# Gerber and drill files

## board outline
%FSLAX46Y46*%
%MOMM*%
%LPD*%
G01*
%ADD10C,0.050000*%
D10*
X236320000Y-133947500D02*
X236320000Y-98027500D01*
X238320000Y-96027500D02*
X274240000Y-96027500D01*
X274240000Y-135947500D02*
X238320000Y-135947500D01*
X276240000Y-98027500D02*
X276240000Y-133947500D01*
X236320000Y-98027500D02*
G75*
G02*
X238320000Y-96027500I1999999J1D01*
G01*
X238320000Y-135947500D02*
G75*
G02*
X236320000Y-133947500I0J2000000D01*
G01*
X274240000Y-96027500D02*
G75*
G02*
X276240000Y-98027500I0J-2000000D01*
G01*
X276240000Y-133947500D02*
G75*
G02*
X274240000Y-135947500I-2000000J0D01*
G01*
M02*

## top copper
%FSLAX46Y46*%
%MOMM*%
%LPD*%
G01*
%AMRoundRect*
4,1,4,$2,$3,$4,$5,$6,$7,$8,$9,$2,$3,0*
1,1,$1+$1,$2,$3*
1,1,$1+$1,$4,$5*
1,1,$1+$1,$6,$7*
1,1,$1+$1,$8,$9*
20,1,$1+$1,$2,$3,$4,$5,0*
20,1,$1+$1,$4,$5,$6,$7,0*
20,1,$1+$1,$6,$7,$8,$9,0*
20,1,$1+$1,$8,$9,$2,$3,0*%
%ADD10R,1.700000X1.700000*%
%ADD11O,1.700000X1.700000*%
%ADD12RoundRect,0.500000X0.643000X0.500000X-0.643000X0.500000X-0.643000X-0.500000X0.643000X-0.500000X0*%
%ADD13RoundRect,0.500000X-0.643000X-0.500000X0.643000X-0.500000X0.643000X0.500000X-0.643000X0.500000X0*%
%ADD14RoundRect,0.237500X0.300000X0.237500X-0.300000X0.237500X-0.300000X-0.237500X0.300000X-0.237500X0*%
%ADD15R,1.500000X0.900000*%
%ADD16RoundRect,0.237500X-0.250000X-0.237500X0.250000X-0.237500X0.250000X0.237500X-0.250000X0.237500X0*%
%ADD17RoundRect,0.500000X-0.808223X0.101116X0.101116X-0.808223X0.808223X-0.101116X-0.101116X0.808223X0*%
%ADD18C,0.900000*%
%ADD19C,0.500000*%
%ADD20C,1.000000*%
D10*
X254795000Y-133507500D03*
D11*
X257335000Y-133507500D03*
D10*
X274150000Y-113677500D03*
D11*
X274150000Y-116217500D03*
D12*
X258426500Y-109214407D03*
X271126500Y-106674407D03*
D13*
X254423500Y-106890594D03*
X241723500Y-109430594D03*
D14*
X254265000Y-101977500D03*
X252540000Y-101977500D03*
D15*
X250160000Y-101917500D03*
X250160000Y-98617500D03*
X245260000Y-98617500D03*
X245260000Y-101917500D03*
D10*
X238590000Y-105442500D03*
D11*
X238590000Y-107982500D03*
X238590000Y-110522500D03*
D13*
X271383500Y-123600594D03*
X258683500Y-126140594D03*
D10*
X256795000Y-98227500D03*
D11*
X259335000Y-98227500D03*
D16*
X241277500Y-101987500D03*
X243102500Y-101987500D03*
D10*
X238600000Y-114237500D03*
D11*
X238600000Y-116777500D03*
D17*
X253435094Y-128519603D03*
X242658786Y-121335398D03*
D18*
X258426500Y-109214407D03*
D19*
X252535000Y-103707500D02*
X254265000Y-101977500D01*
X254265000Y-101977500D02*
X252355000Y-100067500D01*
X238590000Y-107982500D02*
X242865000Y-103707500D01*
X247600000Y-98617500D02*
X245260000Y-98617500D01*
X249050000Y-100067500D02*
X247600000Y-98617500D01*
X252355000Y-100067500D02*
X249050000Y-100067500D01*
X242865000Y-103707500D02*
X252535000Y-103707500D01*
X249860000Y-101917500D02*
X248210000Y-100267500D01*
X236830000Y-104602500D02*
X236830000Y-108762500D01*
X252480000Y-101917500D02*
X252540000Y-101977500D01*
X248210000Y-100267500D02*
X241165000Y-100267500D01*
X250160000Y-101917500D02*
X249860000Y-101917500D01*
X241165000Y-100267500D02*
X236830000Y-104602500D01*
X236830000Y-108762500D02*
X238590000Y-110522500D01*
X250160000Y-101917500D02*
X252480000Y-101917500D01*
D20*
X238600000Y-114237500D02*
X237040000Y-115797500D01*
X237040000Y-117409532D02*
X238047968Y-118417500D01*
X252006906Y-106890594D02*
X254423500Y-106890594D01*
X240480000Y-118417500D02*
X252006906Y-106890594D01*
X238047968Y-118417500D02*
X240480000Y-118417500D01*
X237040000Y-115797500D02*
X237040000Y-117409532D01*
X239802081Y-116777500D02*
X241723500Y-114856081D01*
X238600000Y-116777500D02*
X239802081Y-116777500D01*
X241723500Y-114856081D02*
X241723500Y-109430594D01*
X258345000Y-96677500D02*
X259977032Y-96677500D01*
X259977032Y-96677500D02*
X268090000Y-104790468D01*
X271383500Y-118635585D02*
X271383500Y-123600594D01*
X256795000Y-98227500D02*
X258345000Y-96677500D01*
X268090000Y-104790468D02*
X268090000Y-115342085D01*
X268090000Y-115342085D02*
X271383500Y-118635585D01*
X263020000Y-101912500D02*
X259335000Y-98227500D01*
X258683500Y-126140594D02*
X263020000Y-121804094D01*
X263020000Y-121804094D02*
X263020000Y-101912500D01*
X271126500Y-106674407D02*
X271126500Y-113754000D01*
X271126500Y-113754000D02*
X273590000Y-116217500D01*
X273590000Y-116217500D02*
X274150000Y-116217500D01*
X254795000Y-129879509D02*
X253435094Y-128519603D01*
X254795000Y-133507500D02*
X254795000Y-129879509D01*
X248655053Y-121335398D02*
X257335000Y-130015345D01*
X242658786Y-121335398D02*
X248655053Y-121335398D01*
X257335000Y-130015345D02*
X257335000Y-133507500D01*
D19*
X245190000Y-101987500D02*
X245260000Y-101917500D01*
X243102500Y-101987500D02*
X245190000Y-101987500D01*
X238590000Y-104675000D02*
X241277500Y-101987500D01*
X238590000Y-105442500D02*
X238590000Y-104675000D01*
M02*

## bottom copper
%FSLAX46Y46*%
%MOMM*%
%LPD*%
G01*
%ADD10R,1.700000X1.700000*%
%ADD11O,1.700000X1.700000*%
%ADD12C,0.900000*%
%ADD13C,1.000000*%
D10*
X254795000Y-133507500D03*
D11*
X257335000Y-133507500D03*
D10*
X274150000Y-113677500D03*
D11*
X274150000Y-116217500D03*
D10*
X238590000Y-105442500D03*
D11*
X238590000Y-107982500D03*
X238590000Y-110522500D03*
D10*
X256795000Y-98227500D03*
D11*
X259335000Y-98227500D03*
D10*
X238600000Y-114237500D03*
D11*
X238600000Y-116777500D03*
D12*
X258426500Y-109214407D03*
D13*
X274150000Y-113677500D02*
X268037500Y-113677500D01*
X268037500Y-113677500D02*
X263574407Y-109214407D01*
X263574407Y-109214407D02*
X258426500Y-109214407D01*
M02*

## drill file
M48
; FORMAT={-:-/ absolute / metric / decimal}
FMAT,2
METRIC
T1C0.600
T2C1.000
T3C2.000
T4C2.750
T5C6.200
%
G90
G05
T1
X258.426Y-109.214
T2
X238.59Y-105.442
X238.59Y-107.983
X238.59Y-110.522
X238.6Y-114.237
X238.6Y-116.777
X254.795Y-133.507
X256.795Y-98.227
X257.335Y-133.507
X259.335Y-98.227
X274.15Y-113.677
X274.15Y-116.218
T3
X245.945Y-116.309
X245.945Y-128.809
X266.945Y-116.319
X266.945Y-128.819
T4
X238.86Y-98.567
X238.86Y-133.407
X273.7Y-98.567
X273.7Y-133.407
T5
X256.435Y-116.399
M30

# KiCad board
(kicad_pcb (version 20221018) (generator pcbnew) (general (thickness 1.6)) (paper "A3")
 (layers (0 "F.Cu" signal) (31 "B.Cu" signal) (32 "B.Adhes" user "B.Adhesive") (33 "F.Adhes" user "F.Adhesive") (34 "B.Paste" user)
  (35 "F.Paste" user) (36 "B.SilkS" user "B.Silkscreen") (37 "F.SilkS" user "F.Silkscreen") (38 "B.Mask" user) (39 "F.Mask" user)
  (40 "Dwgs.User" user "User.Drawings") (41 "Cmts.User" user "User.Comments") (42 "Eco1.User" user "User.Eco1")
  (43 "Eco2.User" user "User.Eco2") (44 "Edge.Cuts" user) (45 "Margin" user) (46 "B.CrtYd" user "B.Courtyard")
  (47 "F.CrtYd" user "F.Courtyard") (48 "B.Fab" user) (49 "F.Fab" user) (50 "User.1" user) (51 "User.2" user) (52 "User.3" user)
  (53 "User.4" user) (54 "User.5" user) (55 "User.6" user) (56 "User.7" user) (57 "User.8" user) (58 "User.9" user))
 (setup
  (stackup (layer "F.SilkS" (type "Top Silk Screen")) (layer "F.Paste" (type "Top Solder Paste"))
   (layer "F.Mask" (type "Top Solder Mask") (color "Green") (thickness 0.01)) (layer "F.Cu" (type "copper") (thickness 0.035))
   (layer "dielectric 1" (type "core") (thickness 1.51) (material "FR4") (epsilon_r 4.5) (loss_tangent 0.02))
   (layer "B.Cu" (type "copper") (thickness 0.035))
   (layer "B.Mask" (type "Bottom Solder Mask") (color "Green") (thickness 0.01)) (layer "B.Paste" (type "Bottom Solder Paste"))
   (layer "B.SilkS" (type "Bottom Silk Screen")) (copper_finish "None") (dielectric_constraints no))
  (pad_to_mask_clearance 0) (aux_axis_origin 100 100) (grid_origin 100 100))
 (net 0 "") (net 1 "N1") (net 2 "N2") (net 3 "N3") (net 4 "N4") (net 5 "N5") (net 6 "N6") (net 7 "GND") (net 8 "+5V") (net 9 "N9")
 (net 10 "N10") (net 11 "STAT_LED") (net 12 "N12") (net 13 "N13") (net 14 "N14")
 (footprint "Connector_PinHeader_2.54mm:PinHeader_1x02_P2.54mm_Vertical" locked (layer "F.Cu") (at 254.795 133.5075 90)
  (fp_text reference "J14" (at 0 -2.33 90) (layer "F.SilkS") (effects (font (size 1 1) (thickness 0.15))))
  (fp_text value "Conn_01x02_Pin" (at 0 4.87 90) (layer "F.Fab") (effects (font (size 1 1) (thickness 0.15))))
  (pad "1" thru_hole rect locked (at 0 0 90) (size 1.7 1.7) (drill 1) (layers "*.Cu" "*.Mask") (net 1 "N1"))
  (pad "2" thru_hole oval locked (at 0 2.54 90) (size 1.7 1.7) (drill 1) (layers "*.Cu" "*.Mask") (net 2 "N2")))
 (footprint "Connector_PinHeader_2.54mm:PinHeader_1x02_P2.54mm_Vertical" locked (layer "F.Cu") (at 274.15 113.6775)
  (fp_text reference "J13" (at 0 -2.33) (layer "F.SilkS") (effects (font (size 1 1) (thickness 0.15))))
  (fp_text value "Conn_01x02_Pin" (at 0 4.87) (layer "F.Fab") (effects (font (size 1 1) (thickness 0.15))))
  (pad "1" thru_hole rect locked (at 0 0) (size 1.7 1.7) (drill 1) (layers "*.Cu" "*.Mask") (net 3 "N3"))
  (pad "2" thru_hole oval locked (at 0 2.54) (size 1.7 1.7) (drill 1) (layers "*.Cu" "*.Mask") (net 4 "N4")))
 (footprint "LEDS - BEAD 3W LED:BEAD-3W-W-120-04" (layer "F.Cu") (at 273.6665 104.134407 180)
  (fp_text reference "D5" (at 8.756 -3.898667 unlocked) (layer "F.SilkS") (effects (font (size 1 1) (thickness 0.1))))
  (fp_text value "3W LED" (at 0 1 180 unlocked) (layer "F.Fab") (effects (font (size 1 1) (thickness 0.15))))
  (pad "1" smd roundrect (at 15.24 -5.08 180) (size 2.286 2) (layers "F.Cu" "F.Paste" "F.Mask") (roundrect_rratio 0.25) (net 3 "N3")
   (thermal_bridge_angle 45))
  (pad "2" smd roundrect (at 2.54 -2.54 180) (size 2.286 2) (layers "F.Cu" "F.Paste" "F.Mask") (roundrect_rratio 0.25) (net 4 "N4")
   (thermal_bridge_angle 45)))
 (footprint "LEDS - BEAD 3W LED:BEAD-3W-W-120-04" (layer "F.Cu") (at 239.1835 111.970594)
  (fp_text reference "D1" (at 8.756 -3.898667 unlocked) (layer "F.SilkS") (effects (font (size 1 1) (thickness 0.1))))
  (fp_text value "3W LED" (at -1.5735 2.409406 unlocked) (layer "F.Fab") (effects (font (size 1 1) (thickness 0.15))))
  (pad "1" smd roundrect (at 15.24 -5.08) (size 2.286 2) (layers "F.Cu" "F.Paste" "F.Mask") (roundrect_rratio 0.25) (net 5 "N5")
   (thermal_bridge_angle 45))
  (pad "2" smd roundrect (at 2.54 -2.54) (size 2.286 2) (layers "F.Cu" "F.Paste" "F.Mask") (roundrect_rratio 0.25) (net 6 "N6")
   (thermal_bridge_angle 45)))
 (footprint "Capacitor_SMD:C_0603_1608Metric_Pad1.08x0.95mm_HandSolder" (layer "F.Cu") (at 253.4025 101.9775 180)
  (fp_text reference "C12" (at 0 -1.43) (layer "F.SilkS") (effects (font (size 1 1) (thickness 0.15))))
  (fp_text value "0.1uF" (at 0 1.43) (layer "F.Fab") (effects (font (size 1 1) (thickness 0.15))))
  (pad "1" smd roundrect (at -0.8625 0 180) (size 1.075 0.95) (layers "F.Cu" "F.Paste" "F.Mask") (roundrect_rratio 0.25) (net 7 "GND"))
  (pad "2" smd roundrect (at 0.8625 0 180) (size 1.075 0.95) (layers "F.Cu" "F.Paste" "F.Mask") (roundrect_rratio 0.25) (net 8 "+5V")))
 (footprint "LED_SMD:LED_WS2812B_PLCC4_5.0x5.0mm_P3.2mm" (layer "F.Cu") (at 247.71 100.2675 180)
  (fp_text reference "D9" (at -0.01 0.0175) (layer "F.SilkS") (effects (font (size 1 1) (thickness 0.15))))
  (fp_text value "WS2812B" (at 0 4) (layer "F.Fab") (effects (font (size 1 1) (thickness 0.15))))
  (pad "1" smd rect (at -2.45 -1.65 180) (size 1.5 0.9) (layers "F.Cu" "F.Paste" "F.Mask") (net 8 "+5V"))
  (pad "2" smd rect (at -2.45 1.65 180) (size 1.5 0.9) (layers "F.Cu" "F.Paste" "F.Mask") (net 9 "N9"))
  (pad "3" smd rect (at 2.45 1.65 180) (size 1.5 0.9) (layers "F.Cu" "F.Paste" "F.Mask") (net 7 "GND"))
  (pad "4" smd rect (at 2.45 -1.65 180) (size 1.5 0.9) (layers "F.Cu" "F.Paste" "F.Mask") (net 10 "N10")))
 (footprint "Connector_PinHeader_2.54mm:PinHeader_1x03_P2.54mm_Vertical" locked (layer "F.Cu") (at 238.59 105.4425)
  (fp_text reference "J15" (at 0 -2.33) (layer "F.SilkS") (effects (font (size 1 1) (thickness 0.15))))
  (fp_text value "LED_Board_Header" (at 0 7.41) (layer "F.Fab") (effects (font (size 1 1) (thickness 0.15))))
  (pad "1" thru_hole rect locked (at 0 0) (size 1.7 1.7) (drill 1) (layers "*.Cu" "*.Mask") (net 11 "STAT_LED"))
  (pad "2" thru_hole oval locked (at 0 2.54) (size 1.7 1.7) (drill 1) (layers "*.Cu" "*.Mask") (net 7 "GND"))
  (pad "3" thru_hole oval locked (at 0 5.08) (size 1.7 1.7) (drill 1) (layers "*.Cu" "*.Mask") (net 8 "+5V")))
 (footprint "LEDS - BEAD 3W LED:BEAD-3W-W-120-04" (layer "F.Cu") (at 256.1435 128.680594)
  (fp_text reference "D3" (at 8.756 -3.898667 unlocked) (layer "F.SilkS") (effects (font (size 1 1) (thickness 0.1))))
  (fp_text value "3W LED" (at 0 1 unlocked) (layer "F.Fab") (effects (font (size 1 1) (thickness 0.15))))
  (pad "1" smd roundrect (at 15.24 -5.08) (size 2.286 2) (layers "F.Cu" "F.Paste" "F.Mask") (roundrect_rratio 0.25) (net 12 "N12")
   (thermal_bridge_angle 45))
  (pad "2" smd roundrect (at 2.54 -2.54) (size 2.286 2) (layers "F.Cu" "F.Paste" "F.Mask") (roundrect_rratio 0.25) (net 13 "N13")
   (thermal_bridge_angle 45)))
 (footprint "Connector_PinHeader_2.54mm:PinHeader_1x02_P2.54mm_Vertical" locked (layer "F.Cu") (at 256.795 98.2275 90)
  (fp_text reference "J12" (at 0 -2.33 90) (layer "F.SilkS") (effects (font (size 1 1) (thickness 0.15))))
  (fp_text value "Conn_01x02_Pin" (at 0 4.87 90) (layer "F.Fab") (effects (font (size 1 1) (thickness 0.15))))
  (pad "1" thru_hole rect locked (at 0 0 90) (size 1.7 1.7) (drill 1) (layers "*.Cu" "*.Mask") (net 12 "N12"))
  (pad "2" thru_hole oval locked (at 0 2.54 90) (size 1.7 1.7) (drill 1) (layers "*.Cu" "*.Mask") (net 13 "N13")))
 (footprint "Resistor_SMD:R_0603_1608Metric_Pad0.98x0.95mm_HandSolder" (layer "F.Cu") (at 242.19 101.9875)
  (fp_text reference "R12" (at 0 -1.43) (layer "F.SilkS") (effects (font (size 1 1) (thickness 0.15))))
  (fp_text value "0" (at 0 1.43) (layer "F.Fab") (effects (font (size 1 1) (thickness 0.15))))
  (pad "1" smd roundrect (at -0.9125 0) (size 0.975 0.95) (layers "F.Cu" "F.Paste" "F.Mask") (roundrect_rratio 0.25) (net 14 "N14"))
  (pad "2" smd roundrect (at 0.9125 0) (size 0.975 0.95) (layers "F.Cu" "F.Paste" "F.Mask") (roundrect_rratio 0.25) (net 10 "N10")))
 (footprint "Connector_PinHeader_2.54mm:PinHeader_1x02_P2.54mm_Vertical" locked (layer "F.Cu") (at 238.6 114.2375)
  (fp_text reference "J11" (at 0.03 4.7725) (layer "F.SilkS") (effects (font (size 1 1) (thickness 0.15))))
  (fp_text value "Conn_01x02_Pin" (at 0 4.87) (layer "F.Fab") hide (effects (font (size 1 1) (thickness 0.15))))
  (pad "1" thru_hole rect locked (at 0 0) (size 1.7 1.7) (drill 1) (layers "*.Cu" "*.Mask") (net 5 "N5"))
  (pad "2" thru_hole oval locked (at 0 2.54) (size 1.7 1.7) (drill 1) (layers "*.Cu" "*.Mask") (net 6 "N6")))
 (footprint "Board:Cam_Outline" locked (layer "F.Cu") (at 236.32 96.0275)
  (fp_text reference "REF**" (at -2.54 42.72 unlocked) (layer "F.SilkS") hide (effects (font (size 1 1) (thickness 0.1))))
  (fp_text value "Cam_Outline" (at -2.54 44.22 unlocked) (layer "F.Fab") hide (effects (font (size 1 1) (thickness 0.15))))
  (fp_line (start 0 37.92) (end 0 2) (stroke (width 0.05) (type default)) (layer "Edge.Cuts"))
  (fp_line (start 2 0) (end 37.92 0) (stroke (width 0.05) (type default)) (layer "Edge.Cuts"))
  (fp_line (start 37.92 39.92) (end 2 39.92) (stroke (width 0.05) (type default)) (layer "Edge.Cuts"))
  (fp_line (start 39.92 2) (end 39.92 37.92) (stroke (width 0.05) (type default)) (layer "Edge.Cuts"))
  (fp_arc (start 0 2) (mid 0.585786 0.585786) (end 2 0) (stroke (width 0.05) (type default)) (layer "Edge.Cuts"))
  (fp_arc (start 2 39.92) (mid 0.585786 39.334214) (end 0 37.92) (stroke (width 0.05) (type default)) (layer "Edge.Cuts"))
  (fp_arc (start 37.92 0) (mid 39.334214 0.585786) (end 39.92 2) (stroke (width 0.05) (type default)) (layer "Edge.Cuts"))
  (fp_arc (start 39.92 37.92) (mid 39.334214 39.334214) (end 37.92 39.92) (stroke (width 0.05) (type default)) (layer "Edge.Cuts"))
  (pad "" np_thru_hole circle locked (at 2.54 2.54) (size 2.75 2.75) (drill 2.75) (layers "F&B.Cu" "*.Mask"))
  (pad "" np_thru_hole circle locked (at 2.54 37.38) (size 2.75 2.75) (drill 2.75) (layers "F&B.Cu" "*.Mask"))
  (pad "" np_thru_hole circle locked (at 9.625174 20.281079) (size 2 2) (drill 2) (layers "F&B.Cu" "*.Mask"))
  (pad "" np_thru_hole circle locked (at 9.625174 32.781079) (size 2 2) (drill 2) (layers "F&B.Cu" "*.Mask"))
  (pad "" np_thru_hole circle locked (at 20.115174 20.371079) (size 6.2 6.2) (drill 6.2) (layers "F&B.Cu" "*.Mask"))
  (pad "" np_thru_hole circle locked (at 30.625174 20.291079) (size 2 2) (drill 2) (layers "F&B.Cu" "*.Mask"))
  (pad "" np_thru_hole circle locked (at 30.625174 32.791079) (size 2 2) (drill 2) (layers "F&B.Cu" "*.Mask"))
  (pad "" np_thru_hole circle locked (at 37.38 2.54) (size 2.75 2.75) (drill 2.75) (layers "F&B.Cu" "*.Mask"))
  (pad "" np_thru_hole circle locked (at 37.38 37.38) (size 2.75 2.75) (drill 2.75) (layers "F&B.Cu" "*.Mask")))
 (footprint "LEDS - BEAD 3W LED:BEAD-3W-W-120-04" (layer "F.Cu") (at 239.066684 121.335398 -45)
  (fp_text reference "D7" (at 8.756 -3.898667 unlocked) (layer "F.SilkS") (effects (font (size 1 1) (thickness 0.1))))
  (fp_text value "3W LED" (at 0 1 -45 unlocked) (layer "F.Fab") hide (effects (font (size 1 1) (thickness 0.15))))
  (pad "1" smd roundrect (at 15.24 -5.08 315) (size 2.286 2) (layers "F.Cu" "F.Paste" "F.Mask") (roundrect_rratio 0.25) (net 1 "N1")
   (thermal_bridge_angle 45))
  (pad "2" smd roundrect (at 2.54 -2.54 315) (size 2.286 2) (layers "F.Cu" "F.Paste" "F.Mask") (roundrect_rratio 0.25) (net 2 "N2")
   (thermal_bridge_angle 45)))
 (segment (start 252.535 103.7075) (end 254.265 101.9775) (width 0.5) (layer "F.Cu") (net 7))
 (segment (start 254.265 101.9775) (end 252.355 100.0675) (width 0.5) (layer "F.Cu") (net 7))
 (segment (start 238.59 107.9825) (end 242.865 103.7075) (width 0.5) (layer "F.Cu") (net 7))
 (segment (start 247.6 98.6175) (end 245.26 98.6175) (width 0.5) (layer "F.Cu") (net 7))
 (segment (start 249.05 100.0675) (end 247.6 98.6175) (width 0.5) (layer "F.Cu") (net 7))
 (segment (start 252.355 100.0675) (end 249.05 100.0675) (width 0.5) (layer "F.Cu") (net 7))
 (segment (start 242.865 103.7075) (end 252.535 103.7075) (width 0.5) (layer "F.Cu") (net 7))
 (segment (start 249.86 101.9175) (end 248.21 100.2675) (width 0.5) (layer "F.Cu") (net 8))
 (segment (start 236.83 104.6025) (end 236.83 108.7625) (width 0.5) (layer "F.Cu") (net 8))
 (segment (start 252.48 101.9175) (end 252.54 101.9775) (width 0.5) (layer "F.Cu") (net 8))
 (segment (start 248.21 100.2675) (end 241.165 100.2675) (width 0.5) (layer "F.Cu") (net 8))
 (segment (start 250.16 101.9175) (end 249.86 101.9175) (width 0.5) (layer "F.Cu") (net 8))
 (segment (start 241.165 100.2675) (end 236.83 104.6025) (width 0.5) (layer "F.Cu") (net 8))
 (segment (start 236.83 108.7625) (end 238.59 110.5225) (width 0.5) (layer "F.Cu") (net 8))
 (segment (start 250.16 101.9175) (end 252.48 101.9175) (width 0.5) (layer "F.Cu") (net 8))
 (segment (start 238.6 114.2375) (end 237.04 115.7975) (width 1) (layer "F.Cu") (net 5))
 (segment (start 237.04 117.409532) (end 238.047968 118.4175) (width 1) (layer "F.Cu") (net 5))
 (segment (start 252.006906 106.890594) (end 254.4235 106.890594) (width 1) (layer "F.Cu") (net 5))
 (segment (start 240.48 118.4175) (end 252.006906 106.890594) (width 1) (layer "F.Cu") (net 5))
 (segment (start 238.047968 118.4175) (end 240.48 118.4175) (width 1) (layer "F.Cu") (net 5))
 (segment (start 237.04 115.7975) (end 237.04 117.409532) (width 1) (layer "F.Cu") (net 5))
 (segment (start 239.802081 116.7775) (end 241.7235 114.856081) (width 1) (layer "F.Cu") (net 6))
 (segment (start 238.6 116.7775) (end 239.802081 116.7775) (width 1) (layer "F.Cu") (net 6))
 (segment (start 241.7235 114.856081) (end 241.7235 109.430594) (width 1) (layer "F.Cu") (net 6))
 (segment (start 258.345 96.6775) (end 259.977032 96.6775) (width 1) (layer "F.Cu") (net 12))
 (segment (start 259.977032 96.6775) (end 268.09 104.790468) (width 1) (layer "F.Cu") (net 12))
 (segment (start 271.3835 118.635585) (end 271.3835 123.600594) (width 1) (layer "F.Cu") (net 12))
 (segment (start 256.795 98.2275) (end 258.345 96.6775) (width 1) (layer "F.Cu") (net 12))
 (segment (start 268.09 104.790468) (end 268.09 115.342085) (width 1) (layer "F.Cu") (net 12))
 (segment (start 268.09 115.342085) (end 271.3835 118.635585) (width 1) (layer "F.Cu") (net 12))
 (segment (start 263.02 101.9125) (end 259.335 98.2275) (width 1) (layer "F.Cu") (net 13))
 (segment (start 258.6835 126.140594) (end 263.02 121.804094) (width 1) (layer "F.Cu") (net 13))
 (segment (start 263.02 121.804094) (end 263.02 101.9125) (width 1) (layer "F.Cu") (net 13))
 (via (at 258.4265 109.214407) (size 0.9) (drill 0.6) (layers "F.Cu" "B.Cu") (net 3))
 (segment (start 274.15 113.6775) (end 268.0375 113.6775) (width 1) (layer "B.Cu") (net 3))
 (segment (start 268.0375 113.6775) (end 263.574407 109.214407) (width 1) (layer "B.Cu") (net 3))
 (segment (start 263.574407 109.214407) (end 258.4265 109.214407) (width 1) (layer "B.Cu") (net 3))
 (segment (start 271.1265 106.674407) (end 271.1265 113.754) (width 1) (layer "F.Cu") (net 4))
 (segment (start 271.1265 113.754) (end 273.59 116.2175) (width 1) (layer "F.Cu") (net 4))
 (segment (start 273.59 116.2175) (end 274.15 116.2175) (width 1) (layer "F.Cu") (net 4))
 (segment (start 254.795 129.879509) (end 253.435094 128.519603) (width 1) (layer "F.Cu") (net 1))
 (segment (start 254.795 133.5075) (end 254.795 129.879509) (width 1) (layer "F.Cu") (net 1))
 (segment (start 248.655053 121.335398) (end 257.335 130.015345) (width 1) (layer "F.Cu") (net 2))
 (segment (start 242.658786 121.335398) (end 248.655053 121.335398) (width 1) (layer "F.Cu") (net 2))
 (segment (start 257.335 130.015345) (end 257.335 133.5075) (width 1) (layer "F.Cu") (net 2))
 (segment (start 245.19 101.9875) (end 245.26 101.9175) (width 0.5) (layer "F.Cu") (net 10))
 (segment (start 243.1025 101.9875) (end 245.19 101.9875) (width 0.5) (layer "F.Cu") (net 10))
 (segment (start 238.59 104.675) (end 241.2775 101.9875) (width 0.5) (layer "F.Cu") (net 11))
 (segment (start 238.59 105.4425) (end 238.59 104.675) (width 0.5) (layer "F.Cu") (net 11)))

